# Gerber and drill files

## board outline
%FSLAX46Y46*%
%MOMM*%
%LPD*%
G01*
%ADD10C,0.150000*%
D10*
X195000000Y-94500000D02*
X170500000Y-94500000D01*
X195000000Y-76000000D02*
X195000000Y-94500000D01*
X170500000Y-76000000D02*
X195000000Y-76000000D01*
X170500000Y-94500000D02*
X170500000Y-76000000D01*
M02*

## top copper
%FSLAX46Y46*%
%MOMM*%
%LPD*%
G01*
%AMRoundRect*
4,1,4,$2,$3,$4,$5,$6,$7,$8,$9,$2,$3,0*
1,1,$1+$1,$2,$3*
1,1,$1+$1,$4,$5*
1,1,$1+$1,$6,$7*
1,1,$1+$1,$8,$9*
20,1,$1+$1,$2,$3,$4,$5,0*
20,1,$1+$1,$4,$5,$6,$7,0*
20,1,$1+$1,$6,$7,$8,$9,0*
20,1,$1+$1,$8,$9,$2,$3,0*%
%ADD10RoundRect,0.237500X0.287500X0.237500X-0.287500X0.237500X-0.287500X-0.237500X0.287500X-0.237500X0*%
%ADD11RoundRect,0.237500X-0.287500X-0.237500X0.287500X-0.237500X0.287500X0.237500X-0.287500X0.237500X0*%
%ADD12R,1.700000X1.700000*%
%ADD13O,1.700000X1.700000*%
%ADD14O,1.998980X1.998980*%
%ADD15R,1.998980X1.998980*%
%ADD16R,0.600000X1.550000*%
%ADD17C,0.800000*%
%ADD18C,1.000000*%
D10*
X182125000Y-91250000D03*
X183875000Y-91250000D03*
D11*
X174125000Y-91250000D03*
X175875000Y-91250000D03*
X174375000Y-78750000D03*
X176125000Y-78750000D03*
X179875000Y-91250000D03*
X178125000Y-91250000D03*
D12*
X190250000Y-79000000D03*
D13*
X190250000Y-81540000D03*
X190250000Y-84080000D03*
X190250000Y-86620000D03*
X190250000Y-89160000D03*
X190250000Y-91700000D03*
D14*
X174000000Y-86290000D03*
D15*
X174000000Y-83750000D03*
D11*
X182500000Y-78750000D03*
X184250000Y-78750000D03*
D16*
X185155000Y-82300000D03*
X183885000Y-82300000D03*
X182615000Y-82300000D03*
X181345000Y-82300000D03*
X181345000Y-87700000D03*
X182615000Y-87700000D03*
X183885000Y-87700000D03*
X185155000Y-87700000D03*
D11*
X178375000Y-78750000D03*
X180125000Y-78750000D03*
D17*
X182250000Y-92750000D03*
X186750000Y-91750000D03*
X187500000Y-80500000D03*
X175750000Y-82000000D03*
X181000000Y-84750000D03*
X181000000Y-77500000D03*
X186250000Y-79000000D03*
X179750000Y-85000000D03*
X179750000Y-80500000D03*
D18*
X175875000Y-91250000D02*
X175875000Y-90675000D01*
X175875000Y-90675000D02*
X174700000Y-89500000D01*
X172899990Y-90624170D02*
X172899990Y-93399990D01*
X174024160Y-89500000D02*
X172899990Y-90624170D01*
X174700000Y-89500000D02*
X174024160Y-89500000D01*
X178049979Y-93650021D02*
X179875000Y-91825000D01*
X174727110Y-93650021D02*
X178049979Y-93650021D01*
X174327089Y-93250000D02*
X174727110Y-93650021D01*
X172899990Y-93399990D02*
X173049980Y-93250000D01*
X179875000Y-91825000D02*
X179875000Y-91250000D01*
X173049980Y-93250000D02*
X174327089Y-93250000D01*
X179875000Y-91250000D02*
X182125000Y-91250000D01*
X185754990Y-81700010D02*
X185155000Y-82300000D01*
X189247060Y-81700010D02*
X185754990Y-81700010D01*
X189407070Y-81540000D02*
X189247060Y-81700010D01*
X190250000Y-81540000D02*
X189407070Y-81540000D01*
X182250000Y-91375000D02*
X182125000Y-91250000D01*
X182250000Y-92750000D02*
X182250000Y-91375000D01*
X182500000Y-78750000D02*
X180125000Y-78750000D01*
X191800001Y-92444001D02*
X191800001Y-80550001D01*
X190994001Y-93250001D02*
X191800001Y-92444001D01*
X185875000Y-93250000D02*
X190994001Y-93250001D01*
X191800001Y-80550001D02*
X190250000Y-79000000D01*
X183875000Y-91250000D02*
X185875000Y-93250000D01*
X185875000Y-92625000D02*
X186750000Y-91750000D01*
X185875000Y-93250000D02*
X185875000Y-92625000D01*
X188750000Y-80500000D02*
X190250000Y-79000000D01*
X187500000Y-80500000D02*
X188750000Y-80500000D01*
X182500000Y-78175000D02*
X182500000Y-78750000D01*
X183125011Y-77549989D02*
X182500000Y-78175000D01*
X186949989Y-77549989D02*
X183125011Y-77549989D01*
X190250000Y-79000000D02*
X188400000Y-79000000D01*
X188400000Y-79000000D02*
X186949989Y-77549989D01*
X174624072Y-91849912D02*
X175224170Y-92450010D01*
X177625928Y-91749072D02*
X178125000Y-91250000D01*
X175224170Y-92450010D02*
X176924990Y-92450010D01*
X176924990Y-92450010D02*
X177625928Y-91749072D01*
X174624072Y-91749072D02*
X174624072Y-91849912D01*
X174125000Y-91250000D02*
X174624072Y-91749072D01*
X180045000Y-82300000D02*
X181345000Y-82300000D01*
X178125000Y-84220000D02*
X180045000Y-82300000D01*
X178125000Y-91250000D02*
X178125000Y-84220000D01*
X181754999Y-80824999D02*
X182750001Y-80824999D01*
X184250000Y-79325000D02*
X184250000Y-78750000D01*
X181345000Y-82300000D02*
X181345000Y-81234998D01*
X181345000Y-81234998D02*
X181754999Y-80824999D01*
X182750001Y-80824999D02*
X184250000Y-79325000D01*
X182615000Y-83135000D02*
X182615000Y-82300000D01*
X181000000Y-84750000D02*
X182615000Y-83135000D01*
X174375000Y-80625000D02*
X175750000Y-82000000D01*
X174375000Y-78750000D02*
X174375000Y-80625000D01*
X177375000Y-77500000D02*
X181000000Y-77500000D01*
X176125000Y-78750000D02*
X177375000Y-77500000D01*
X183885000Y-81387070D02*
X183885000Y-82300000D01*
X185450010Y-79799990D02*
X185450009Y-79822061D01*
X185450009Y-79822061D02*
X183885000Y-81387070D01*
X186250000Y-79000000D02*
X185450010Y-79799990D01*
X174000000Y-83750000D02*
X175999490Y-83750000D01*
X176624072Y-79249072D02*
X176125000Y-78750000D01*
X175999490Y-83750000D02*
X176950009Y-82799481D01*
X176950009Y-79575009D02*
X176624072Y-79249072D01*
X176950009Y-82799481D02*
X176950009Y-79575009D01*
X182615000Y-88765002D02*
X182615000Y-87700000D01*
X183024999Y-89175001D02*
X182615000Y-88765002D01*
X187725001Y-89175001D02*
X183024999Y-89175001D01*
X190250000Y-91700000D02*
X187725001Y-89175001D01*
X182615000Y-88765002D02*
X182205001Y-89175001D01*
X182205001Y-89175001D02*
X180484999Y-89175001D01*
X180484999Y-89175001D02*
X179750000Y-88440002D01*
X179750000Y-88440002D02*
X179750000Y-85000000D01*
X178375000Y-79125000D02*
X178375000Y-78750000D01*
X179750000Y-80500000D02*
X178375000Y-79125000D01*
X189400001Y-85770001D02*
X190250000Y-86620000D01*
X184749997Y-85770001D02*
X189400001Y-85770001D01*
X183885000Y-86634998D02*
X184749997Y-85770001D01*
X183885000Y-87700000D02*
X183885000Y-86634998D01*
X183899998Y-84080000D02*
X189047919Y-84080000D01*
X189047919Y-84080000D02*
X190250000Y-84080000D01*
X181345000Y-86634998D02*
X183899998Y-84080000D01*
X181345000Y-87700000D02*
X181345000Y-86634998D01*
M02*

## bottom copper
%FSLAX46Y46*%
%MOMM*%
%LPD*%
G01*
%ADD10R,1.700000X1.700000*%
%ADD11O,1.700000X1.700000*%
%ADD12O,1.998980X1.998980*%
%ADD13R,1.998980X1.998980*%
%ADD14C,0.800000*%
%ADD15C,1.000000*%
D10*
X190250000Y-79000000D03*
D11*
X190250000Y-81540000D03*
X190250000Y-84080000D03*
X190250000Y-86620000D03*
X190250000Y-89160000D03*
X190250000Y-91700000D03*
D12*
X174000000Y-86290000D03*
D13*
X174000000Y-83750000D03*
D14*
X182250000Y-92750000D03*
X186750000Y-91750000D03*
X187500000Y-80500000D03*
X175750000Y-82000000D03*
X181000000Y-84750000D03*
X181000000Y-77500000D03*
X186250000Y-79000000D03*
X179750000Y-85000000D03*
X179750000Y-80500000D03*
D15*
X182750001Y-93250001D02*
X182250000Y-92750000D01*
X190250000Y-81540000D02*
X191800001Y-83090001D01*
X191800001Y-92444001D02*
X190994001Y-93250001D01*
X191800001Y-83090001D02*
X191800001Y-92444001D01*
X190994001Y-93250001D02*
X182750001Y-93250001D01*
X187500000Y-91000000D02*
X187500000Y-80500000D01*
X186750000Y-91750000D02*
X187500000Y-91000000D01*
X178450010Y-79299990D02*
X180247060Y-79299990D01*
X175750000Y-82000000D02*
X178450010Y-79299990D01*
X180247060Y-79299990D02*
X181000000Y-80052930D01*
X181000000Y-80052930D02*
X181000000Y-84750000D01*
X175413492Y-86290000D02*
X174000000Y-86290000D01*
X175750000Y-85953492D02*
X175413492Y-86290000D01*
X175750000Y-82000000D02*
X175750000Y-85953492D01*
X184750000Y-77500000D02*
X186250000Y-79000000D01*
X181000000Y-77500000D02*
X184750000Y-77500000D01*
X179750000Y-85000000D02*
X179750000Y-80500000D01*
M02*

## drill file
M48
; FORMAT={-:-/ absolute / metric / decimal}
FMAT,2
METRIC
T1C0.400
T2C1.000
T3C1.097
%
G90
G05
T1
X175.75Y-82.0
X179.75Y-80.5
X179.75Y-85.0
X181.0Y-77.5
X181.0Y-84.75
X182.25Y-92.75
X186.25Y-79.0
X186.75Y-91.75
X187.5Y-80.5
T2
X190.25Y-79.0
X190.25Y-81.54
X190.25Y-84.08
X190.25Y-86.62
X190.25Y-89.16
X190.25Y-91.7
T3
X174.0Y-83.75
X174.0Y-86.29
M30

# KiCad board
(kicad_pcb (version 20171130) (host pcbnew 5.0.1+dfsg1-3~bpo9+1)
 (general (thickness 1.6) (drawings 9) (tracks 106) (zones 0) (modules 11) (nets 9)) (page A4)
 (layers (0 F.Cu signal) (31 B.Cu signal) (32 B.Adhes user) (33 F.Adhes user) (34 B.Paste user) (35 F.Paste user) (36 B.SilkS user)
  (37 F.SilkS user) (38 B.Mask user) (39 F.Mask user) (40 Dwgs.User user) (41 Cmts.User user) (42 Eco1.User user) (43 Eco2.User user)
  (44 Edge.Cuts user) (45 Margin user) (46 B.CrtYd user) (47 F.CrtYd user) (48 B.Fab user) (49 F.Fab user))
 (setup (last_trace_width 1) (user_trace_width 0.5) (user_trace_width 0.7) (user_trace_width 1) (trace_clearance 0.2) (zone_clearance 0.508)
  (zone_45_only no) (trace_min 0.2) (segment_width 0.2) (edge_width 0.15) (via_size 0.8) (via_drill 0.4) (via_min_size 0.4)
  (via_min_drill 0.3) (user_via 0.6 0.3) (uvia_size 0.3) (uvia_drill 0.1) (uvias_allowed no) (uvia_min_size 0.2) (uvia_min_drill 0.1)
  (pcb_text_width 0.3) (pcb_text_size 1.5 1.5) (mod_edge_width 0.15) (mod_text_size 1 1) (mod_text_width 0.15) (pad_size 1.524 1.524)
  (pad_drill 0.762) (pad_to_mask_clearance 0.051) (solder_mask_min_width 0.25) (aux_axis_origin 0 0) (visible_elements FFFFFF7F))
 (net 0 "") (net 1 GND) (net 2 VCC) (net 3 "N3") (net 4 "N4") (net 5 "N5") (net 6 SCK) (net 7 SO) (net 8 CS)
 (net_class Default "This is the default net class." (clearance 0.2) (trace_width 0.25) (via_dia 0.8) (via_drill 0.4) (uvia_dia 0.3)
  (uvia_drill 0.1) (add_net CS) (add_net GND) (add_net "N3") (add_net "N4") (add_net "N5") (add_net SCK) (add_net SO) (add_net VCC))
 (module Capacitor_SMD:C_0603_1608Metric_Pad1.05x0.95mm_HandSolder (layer F.Cu) (at 183 91.25 180)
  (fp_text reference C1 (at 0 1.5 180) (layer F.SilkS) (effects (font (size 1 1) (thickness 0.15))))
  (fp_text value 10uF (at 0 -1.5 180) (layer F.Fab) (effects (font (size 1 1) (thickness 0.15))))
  (pad 2 smd roundrect (at 0.875 0 180) (size 1.05 0.95) (layers F.Cu F.Paste F.Mask) (roundrect_rratio 0.25) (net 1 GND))
  (pad 1 smd roundrect (at -0.875 0 180) (size 1.05 0.95) (layers F.Cu F.Paste F.Mask) (roundrect_rratio 0.25) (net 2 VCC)))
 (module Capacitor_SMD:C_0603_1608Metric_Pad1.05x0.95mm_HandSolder (layer F.Cu) (at 175 91.25)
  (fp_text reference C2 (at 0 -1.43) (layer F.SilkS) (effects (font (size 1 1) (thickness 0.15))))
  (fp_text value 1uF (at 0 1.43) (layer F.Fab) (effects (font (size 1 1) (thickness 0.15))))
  (pad 1 smd roundrect (at -0.875 0) (size 1.05 0.95) (layers F.Cu F.Paste F.Mask) (roundrect_rratio 0.25) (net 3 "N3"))
  (pad 2 smd roundrect (at 0.875 0) (size 1.05 0.95) (layers F.Cu F.Paste F.Mask) (roundrect_rratio 0.25) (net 1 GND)))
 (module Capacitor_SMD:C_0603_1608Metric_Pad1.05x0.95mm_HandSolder (layer F.Cu) (at 175.25 78.75)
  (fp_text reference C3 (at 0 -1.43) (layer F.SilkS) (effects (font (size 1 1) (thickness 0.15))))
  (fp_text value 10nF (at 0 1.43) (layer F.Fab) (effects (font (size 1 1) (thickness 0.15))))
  (pad 1 smd roundrect (at -0.875 0) (size 1.05 0.95) (layers F.Cu F.Paste F.Mask) (roundrect_rratio 0.25) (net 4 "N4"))
  (pad 2 smd roundrect (at 0.875 0) (size 1.05 0.95) (layers F.Cu F.Paste F.Mask) (roundrect_rratio 0.25) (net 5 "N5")))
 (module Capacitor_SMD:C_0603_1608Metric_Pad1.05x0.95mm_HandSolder (layer F.Cu) (at 179 91.25)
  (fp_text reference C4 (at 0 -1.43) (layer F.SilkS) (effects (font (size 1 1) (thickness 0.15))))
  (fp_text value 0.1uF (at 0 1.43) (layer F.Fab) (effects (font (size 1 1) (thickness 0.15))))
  (pad 2 smd roundrect (at 0.875 0) (size 1.05 0.95) (layers F.Cu F.Paste F.Mask) (roundrect_rratio 0.25) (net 1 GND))
  (pad 1 smd roundrect (at -0.875 0) (size 1.05 0.95) (layers F.Cu F.Paste F.Mask) (roundrect_rratio 0.25) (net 3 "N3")))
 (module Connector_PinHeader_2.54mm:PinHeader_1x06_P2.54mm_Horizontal (layer F.Cu) (at 190.25 79)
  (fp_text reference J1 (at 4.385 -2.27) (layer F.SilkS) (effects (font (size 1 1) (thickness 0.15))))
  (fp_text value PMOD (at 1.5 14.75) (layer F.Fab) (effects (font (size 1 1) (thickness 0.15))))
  (pad 1 thru_hole rect (at 0 0) (size 1.7 1.7) (drill 1) (layers *.Cu *.Mask) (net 2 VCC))
  (pad 2 thru_hole oval (at 0 2.54) (size 1.7 1.7) (drill 1) (layers *.Cu *.Mask) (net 1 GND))
  (pad 3 thru_hole oval (at 0 5.08) (size 1.7 1.7) (drill 1) (layers *.Cu *.Mask) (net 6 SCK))
  (pad 4 thru_hole oval (at 0 7.62) (size 1.7 1.7) (drill 1) (layers *.Cu *.Mask) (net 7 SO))
  (pad 5 thru_hole oval (at 0 10.16) (size 1.7 1.7) (drill 1) (layers *.Cu *.Mask))
  (pad 6 thru_hole oval (at 0 12.7) (size 1.7 1.7) (drill 1) (layers *.Cu *.Mask) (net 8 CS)))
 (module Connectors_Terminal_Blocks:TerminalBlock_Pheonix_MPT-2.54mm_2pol (layer F.Cu) (at 174 83.75 270)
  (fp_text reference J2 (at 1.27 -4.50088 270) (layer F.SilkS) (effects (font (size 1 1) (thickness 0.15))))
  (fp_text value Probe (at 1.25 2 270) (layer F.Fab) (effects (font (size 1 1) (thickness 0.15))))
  (pad 2 thru_hole oval (at 2.54 0 270) (size 1.99898 1.99898) (drill 1.09728) (layers *.Cu *.Mask) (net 4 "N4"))
  (pad 1 thru_hole rect (at 0 0 270) (size 1.99898 1.99898) (drill 1.09728) (layers *.Cu *.Mask) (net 5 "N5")))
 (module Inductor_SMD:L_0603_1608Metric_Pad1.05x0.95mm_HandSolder (layer F.Cu) (at 183.375 78.75)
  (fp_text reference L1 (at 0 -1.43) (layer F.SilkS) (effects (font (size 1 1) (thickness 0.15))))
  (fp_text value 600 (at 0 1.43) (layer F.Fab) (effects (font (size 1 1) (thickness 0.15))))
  (pad 1 smd roundrect (at -0.875 0) (size 1.05 0.95) (layers F.Cu F.Paste F.Mask) (roundrect_rratio 0.25) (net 2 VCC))
  (pad 2 smd roundrect (at 0.875 0) (size 1.05 0.95) (layers F.Cu F.Paste F.Mask) (roundrect_rratio 0.25) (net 3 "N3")))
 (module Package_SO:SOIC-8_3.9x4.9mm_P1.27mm (layer F.Cu) (at 183.25 85 270)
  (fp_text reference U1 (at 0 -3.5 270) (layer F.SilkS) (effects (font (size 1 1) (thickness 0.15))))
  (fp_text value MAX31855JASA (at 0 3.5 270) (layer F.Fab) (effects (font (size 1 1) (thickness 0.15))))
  (pad 1 smd rect (at -2.7 -1.905 270) (size 1.55 0.6) (layers F.Cu F.Paste F.Mask) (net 1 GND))
  (pad 2 smd rect (at -2.7 -0.635 270) (size 1.55 0.6) (layers F.Cu F.Paste F.Mask) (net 5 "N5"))
  (pad 3 smd rect (at -2.7 0.635 270) (size 1.55 0.6) (layers F.Cu F.Paste F.Mask) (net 4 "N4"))
  (pad 4 smd rect (at -2.7 1.905 270) (size 1.55 0.6) (layers F.Cu F.Paste F.Mask) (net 3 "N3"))
  (pad 5 smd rect (at 2.7 1.905 270) (size 1.55 0.6) (layers F.Cu F.Paste F.Mask) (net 6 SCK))
  (pad 6 smd rect (at 2.7 0.635 270) (size 1.55 0.6) (layers F.Cu F.Paste F.Mask) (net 8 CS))
  (pad 7 smd rect (at 2.7 -0.635 270) (size 1.55 0.6) (layers F.Cu F.Paste F.Mask) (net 7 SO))
  (pad 8 smd rect (at 2.7 -1.905 270) (size 1.55 0.6) (layers F.Cu F.Paste F.Mask)))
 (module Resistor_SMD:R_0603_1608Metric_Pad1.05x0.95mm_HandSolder (layer F.Cu) (at 179.25 78.75)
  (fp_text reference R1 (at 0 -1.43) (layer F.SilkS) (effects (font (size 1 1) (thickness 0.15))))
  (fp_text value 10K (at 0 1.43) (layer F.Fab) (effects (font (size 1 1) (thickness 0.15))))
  (pad 1 smd roundrect (at -0.875 0) (size 1.05 0.95) (layers F.Cu F.Paste F.Mask) (roundrect_rratio 0.25) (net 8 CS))
  (pad 2 smd roundrect (at 0.875 0) (size 1.05 0.95) (layers F.Cu F.Paste F.Mask) (roundrect_rratio 0.25) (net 2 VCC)))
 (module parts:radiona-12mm (layer B.Cu) (at 181 78.5)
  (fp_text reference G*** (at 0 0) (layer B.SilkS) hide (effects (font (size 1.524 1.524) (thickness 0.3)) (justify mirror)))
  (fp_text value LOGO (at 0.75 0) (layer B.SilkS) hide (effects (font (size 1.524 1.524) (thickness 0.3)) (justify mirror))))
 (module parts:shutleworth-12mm (layer B.Cu) (at 180.5 92.25)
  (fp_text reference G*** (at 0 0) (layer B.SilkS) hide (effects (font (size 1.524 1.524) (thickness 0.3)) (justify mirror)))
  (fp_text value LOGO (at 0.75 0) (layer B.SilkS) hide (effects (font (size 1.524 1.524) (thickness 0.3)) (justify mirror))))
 (gr_line (start 195 94.5) (end 170.5 94.5) (layer Edge.Cuts) (width 0.15))
 (gr_line (start 195 76) (end 195 94.5) (layer Edge.Cuts) (width 0.15))
 (gr_line (start 170.5 76) (end 195 76) (layer Edge.Cuts) (width 0.15))
 (gr_line (start 170.5 94.5) (end 170.5 76) (layer Edge.Cuts) (width 0.15))
 (segment (start 175.875 91.25) (end 175.875 90.675) (width 1) (layer F.Cu) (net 1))
 (segment (start 175.875 90.675) (end 174.7 89.5) (width 1) (layer F.Cu) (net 1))
 (segment (start 172.89999 90.62417) (end 172.89999 93.39999) (width 1) (layer F.Cu) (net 1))
 (segment (start 174.02416 89.5) (end 172.89999 90.62417) (width 1) (layer F.Cu) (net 1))
 (segment (start 174.7 89.5) (end 174.02416 89.5) (width 1) (layer F.Cu) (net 1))
 (segment (start 178.049979 93.650021) (end 179.875 91.825) (width 1) (layer F.Cu) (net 1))
 (segment (start 174.72711 93.650021) (end 178.049979 93.650021) (width 1) (layer F.Cu) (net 1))
 (segment (start 174.327089 93.25) (end 174.72711 93.650021) (width 1) (layer F.Cu) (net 1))
 (segment (start 172.89999 93.39999) (end 173.04998 93.25) (width 1) (layer F.Cu) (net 1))
 (segment (start 179.875 91.825) (end 179.875 91.25) (width 1) (layer F.Cu) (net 1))
 (segment (start 173.04998 93.25) (end 174.327089 93.25) (width 1) (layer F.Cu) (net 1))
 (segment (start 179.875 91.25) (end 182.125 91.25) (width 1) (layer F.Cu) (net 1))
 (segment (start 185.75499 81.70001) (end 185.155 82.3) (width 1) (layer F.Cu) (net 1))
 (segment (start 189.24706 81.70001) (end 185.75499 81.70001) (width 1) (layer F.Cu) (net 1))
 (segment (start 189.40707 81.54) (end 189.24706 81.70001) (width 1) (layer F.Cu) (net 1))
 (segment (start 190.25 81.54) (end 189.40707 81.54) (width 1) (layer F.Cu) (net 1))
 (via (at 182.25 92.75) (size 0.8) (drill 0.4) (layers F.Cu B.Cu) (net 1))
 (segment (start 182.750001 93.250001) (end 182.25 92.75) (width 1) (layer B.Cu) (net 1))
 (segment (start 190.25 81.54) (end 191.800001 83.090001) (width 1) (layer B.Cu) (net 1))
 (segment (start 191.800001 92.444001) (end 190.994001 93.250001) (width 1) (layer B.Cu) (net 1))
 (segment (start 191.800001 83.090001) (end 191.800001 92.444001) (width 1) (layer B.Cu) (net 1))
 (segment (start 190.994001 93.250001) (end 182.750001 93.250001) (width 1) (layer B.Cu) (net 1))
 (segment (start 182.25 91.375) (end 182.125 91.25) (width 1) (layer F.Cu) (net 1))
 (segment (start 182.25 92.75) (end 182.25 91.375) (width 1) (layer F.Cu) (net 1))
 (segment (start 182.5 78.75) (end 180.125 78.75) (width 1) (layer F.Cu) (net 2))
 (segment (start 191.800001 92.444001) (end 191.800001 80.550001) (width 1) (layer F.Cu) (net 2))
 (segment (start 190.994001 93.250001) (end 191.800001 92.444001) (width 1) (layer F.Cu) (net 2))
 (segment (start 185.875 93.25) (end 190.994001 93.250001) (width 1) (layer F.Cu) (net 2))
 (segment (start 191.800001 80.550001) (end 190.25 79) (width 1) (layer F.Cu) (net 2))
 (segment (start 183.875 91.25) (end 185.875 93.25) (width 1) (layer F.Cu) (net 2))
 (via (at 186.75 91.75) (size 0.8) (drill 0.4) (layers F.Cu B.Cu) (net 2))
 (segment (start 185.875 92.625) (end 186.75 91.75) (width 1) (layer F.Cu) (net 2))
 (segment (start 185.875 93.25) (end 185.875 92.625) (width 1) (layer F.Cu) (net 2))
 (via (at 187.5 80.5) (size 0.8) (drill 0.4) (layers F.Cu B.Cu) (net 2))
 (segment (start 187.5 91) (end 187.5 80.5) (width 1) (layer B.Cu) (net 2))
 (segment (start 186.75 91.75) (end 187.5 91) (width 1) (layer B.Cu) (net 2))
 (segment (start 188.75 80.5) (end 190.25 79) (width 1) (layer F.Cu) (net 2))
 (segment (start 187.5 80.5) (end 188.75 80.5) (width 1) (layer F.Cu) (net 2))
 (segment (start 182.5 78.175) (end 182.5 78.75) (width 1) (layer F.Cu) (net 2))
 (segment (start 183.125011 77.549989) (end 182.5 78.175) (width 1) (layer F.Cu) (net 2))
 (segment (start 186.949989 77.549989) (end 183.125011 77.549989) (width 1) (layer F.Cu) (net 2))
 (segment (start 190.25 79) (end 188.4 79) (width 1) (layer F.Cu) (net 2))
 (segment (start 188.4 79) (end 186.949989 77.549989) (width 1) (layer F.Cu) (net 2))
 (segment (start 174.624072 91.849912) (end 175.22417 92.45001) (width 1) (layer F.Cu) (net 3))
 (segment (start 177.625928 91.749072) (end 178.125 91.25) (width 1) (layer F.Cu) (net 3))
 (segment (start 175.22417 92.45001) (end 176.92499 92.45001) (width 1) (layer F.Cu) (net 3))
 (segment (start 176.92499 92.45001) (end 177.625928 91.749072) (width 1) (layer F.Cu) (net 3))
 (segment (start 174.624072 91.749072) (end 174.624072 91.849912) (width 1) (layer F.Cu) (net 3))
 (segment (start 174.125 91.25) (end 174.624072 91.749072) (width 1) (layer F.Cu) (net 3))
 (segment (start 180.045 82.3) (end 181.345 82.3) (width 1) (layer F.Cu) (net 3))
 (segment (start 178.125 84.22) (end 180.045 82.3) (width 1) (layer F.Cu) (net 3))
 (segment (start 178.125 91.25) (end 178.125 84.22) (width 1) (layer F.Cu) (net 3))
 (segment (start 181.754999 80.824999) (end 182.750001 80.824999) (width 1) (layer F.Cu) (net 3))
 (segment (start 184.25 79.325) (end 184.25 78.75) (width 1) (layer F.Cu) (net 3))
 (segment (start 181.345 82.3) (end 181.345 81.234998) (width 1) (layer F.Cu) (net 3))
 (segment (start 181.345 81.234998) (end 181.754999 80.824999) (width 1) (layer F.Cu) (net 3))
 (segment (start 182.750001 80.824999) (end 184.25 79.325) (width 1) (layer F.Cu) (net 3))
 (via (at 175.75 82) (size 0.8) (drill 0.4) (layers F.Cu B.Cu) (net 4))
 (via (at 181 84.75) (size 0.8) (drill 0.4) (layers F.Cu B.Cu) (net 4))
 (segment (start 178.45001 79.29999) (end 180.24706 79.29999) (width 1) (layer B.Cu) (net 4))
 (segment (start 175.75 82) (end 178.45001 79.29999) (width 1) (layer B.Cu) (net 4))
 (segment (start 180.24706 79.29999) (end 181 80.05293) (width 1) (layer B.Cu) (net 4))
 (segment (start 181 80.05293) (end 181 84.75) (width 1) (layer B.Cu) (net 4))
 (segment (start 182.615 83.135) (end 182.615 82.3) (width 1) (layer F.Cu) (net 4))
 (segment (start 181 84.75) (end 182.615 83.135) (width 1) (layer F.Cu) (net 4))
 (segment (start 174.375 80.625) (end 175.75 82) (width 1) (layer F.Cu) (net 4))
 (segment (start 174.375 78.75) (end 174.375 80.625) (width 1) (layer F.Cu) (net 4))
 (segment (start 175.413492 86.29) (end 174 86.29) (width 1) (layer B.Cu) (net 4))
 (segment (start 175.75 85.953492) (end 175.413492 86.29) (width 1) (layer B.Cu) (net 4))
 (segment (start 175.75 82) (end 175.75 85.953492) (width 1) (layer B.Cu) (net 4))
 (segment (start 177.375 77.5) (end 181 77.5) (width 1) (layer F.Cu) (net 5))
 (via (at 181 77.5) (size 0.8) (drill 0.4) (layers F.Cu B.Cu) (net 5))
 (segment (start 176.125 78.75) (end 177.375 77.5) (width 1) (layer F.Cu) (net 5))
 (via (at 186.25 79) (size 0.8) (drill 0.4) (layers F.Cu B.Cu) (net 5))
 (segment (start 184.75 77.5) (end 186.25 79) (width 1) (layer B.Cu) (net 5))
 (segment (start 181 77.5) (end 184.75 77.5) (width 1) (layer B.Cu) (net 5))
 (segment (start 183.885 81.38707) (end 183.885 82.3) (width 1) (layer F.Cu) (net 5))
 (segment (start 185.45001 79.79999) (end 185.450009 79.822061) (width 1) (layer F.Cu) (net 5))
 (segment (start 185.450009 79.822061) (end 183.885 81.38707) (width 1) (layer F.Cu) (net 5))
 (segment (start 186.25 79) (end 185.45001 79.79999) (width 1) (layer F.Cu) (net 5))
 (segment (start 174 83.75) (end 175.99949 83.75) (width 1) (layer F.Cu) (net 5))
 (segment (start 176.624072 79.249072) (end 176.125 78.75) (width 1) (layer F.Cu) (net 5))
 (segment (start 175.99949 83.75) (end 176.950009 82.799481) (width 1) (layer F.Cu) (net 5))
 (segment (start 176.950009 79.575009) (end 176.624072 79.249072) (width 1) (layer F.Cu) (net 5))
 (segment (start 176.950009 82.799481) (end 176.950009 79.575009) (width 1) (layer F.Cu) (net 5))
 (segment (start 182.615 88.765002) (end 182.615 87.7) (width 1) (layer F.Cu) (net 8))
 (segment (start 183.024999 89.175001) (end 182.615 88.765002) (width 1) (layer F.Cu) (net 8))
 (segment (start 187.725001 89.175001) (end 183.024999 89.175001) (width 1) (layer F.Cu) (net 8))
 (segment (start 190.25 91.7) (end 187.725001 89.175001) (width 1) (layer F.Cu) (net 8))
 (via (at 179.75 85) (size 0.8) (drill 0.4) (layers F.Cu B.Cu) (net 8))
 (segment (start 182.615 88.765002) (end 182.205001 89.175001) (width 1) (layer F.Cu) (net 8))
 (segment (start 182.205001 89.175001) (end 180.484999 89.175001) (width 1) (layer F.Cu) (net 8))
 (segment (start 180.484999 89.175001) (end 179.75 88.440002) (width 1) (layer F.Cu) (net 8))
 (segment (start 179.75 88.440002) (end 179.75 85) (width 1) (layer F.Cu) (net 8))
 (via (at 179.75 80.5) (size 0.8) (drill 0.4) (layers F.Cu B.Cu) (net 8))
 (segment (start 179.75 85) (end 179.75 80.5) (width 1) (layer B.Cu) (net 8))
 (segment (start 178.375 79.125) (end 178.375 78.75) (width 1) (layer F.Cu) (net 8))
 (segment (start 179.75 80.5) (end 178.375 79.125) (width 1) (layer F.Cu) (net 8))
 (segment (start 189.400001 85.770001) (end 190.25 86.62) (width 1) (layer F.Cu) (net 7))
 (segment (start 184.749997 85.770001) (end 189.400001 85.770001) (width 1) (layer F.Cu) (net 7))
 (segment (start 183.885 86.634998) (end 184.749997 85.770001) (width 1) (layer F.Cu) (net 7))
 (segment (start 183.885 87.7) (end 183.885 86.634998) (width 1) (layer F.Cu) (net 7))
 (segment (start 183.899998 84.08) (end 189.047919 84.08) (width 1) (layer F.Cu) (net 6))
 (segment (start 189.047919 84.08) (end 190.25 84.08) (width 1) (layer F.Cu) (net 6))
 (segment (start 181.345 86.634998) (end 183.899998 84.08) (width 1) (layer F.Cu) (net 6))
 (segment (start 181.345 87.7) (end 181.345 86.634998) (width 1) (layer F.Cu) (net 6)))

